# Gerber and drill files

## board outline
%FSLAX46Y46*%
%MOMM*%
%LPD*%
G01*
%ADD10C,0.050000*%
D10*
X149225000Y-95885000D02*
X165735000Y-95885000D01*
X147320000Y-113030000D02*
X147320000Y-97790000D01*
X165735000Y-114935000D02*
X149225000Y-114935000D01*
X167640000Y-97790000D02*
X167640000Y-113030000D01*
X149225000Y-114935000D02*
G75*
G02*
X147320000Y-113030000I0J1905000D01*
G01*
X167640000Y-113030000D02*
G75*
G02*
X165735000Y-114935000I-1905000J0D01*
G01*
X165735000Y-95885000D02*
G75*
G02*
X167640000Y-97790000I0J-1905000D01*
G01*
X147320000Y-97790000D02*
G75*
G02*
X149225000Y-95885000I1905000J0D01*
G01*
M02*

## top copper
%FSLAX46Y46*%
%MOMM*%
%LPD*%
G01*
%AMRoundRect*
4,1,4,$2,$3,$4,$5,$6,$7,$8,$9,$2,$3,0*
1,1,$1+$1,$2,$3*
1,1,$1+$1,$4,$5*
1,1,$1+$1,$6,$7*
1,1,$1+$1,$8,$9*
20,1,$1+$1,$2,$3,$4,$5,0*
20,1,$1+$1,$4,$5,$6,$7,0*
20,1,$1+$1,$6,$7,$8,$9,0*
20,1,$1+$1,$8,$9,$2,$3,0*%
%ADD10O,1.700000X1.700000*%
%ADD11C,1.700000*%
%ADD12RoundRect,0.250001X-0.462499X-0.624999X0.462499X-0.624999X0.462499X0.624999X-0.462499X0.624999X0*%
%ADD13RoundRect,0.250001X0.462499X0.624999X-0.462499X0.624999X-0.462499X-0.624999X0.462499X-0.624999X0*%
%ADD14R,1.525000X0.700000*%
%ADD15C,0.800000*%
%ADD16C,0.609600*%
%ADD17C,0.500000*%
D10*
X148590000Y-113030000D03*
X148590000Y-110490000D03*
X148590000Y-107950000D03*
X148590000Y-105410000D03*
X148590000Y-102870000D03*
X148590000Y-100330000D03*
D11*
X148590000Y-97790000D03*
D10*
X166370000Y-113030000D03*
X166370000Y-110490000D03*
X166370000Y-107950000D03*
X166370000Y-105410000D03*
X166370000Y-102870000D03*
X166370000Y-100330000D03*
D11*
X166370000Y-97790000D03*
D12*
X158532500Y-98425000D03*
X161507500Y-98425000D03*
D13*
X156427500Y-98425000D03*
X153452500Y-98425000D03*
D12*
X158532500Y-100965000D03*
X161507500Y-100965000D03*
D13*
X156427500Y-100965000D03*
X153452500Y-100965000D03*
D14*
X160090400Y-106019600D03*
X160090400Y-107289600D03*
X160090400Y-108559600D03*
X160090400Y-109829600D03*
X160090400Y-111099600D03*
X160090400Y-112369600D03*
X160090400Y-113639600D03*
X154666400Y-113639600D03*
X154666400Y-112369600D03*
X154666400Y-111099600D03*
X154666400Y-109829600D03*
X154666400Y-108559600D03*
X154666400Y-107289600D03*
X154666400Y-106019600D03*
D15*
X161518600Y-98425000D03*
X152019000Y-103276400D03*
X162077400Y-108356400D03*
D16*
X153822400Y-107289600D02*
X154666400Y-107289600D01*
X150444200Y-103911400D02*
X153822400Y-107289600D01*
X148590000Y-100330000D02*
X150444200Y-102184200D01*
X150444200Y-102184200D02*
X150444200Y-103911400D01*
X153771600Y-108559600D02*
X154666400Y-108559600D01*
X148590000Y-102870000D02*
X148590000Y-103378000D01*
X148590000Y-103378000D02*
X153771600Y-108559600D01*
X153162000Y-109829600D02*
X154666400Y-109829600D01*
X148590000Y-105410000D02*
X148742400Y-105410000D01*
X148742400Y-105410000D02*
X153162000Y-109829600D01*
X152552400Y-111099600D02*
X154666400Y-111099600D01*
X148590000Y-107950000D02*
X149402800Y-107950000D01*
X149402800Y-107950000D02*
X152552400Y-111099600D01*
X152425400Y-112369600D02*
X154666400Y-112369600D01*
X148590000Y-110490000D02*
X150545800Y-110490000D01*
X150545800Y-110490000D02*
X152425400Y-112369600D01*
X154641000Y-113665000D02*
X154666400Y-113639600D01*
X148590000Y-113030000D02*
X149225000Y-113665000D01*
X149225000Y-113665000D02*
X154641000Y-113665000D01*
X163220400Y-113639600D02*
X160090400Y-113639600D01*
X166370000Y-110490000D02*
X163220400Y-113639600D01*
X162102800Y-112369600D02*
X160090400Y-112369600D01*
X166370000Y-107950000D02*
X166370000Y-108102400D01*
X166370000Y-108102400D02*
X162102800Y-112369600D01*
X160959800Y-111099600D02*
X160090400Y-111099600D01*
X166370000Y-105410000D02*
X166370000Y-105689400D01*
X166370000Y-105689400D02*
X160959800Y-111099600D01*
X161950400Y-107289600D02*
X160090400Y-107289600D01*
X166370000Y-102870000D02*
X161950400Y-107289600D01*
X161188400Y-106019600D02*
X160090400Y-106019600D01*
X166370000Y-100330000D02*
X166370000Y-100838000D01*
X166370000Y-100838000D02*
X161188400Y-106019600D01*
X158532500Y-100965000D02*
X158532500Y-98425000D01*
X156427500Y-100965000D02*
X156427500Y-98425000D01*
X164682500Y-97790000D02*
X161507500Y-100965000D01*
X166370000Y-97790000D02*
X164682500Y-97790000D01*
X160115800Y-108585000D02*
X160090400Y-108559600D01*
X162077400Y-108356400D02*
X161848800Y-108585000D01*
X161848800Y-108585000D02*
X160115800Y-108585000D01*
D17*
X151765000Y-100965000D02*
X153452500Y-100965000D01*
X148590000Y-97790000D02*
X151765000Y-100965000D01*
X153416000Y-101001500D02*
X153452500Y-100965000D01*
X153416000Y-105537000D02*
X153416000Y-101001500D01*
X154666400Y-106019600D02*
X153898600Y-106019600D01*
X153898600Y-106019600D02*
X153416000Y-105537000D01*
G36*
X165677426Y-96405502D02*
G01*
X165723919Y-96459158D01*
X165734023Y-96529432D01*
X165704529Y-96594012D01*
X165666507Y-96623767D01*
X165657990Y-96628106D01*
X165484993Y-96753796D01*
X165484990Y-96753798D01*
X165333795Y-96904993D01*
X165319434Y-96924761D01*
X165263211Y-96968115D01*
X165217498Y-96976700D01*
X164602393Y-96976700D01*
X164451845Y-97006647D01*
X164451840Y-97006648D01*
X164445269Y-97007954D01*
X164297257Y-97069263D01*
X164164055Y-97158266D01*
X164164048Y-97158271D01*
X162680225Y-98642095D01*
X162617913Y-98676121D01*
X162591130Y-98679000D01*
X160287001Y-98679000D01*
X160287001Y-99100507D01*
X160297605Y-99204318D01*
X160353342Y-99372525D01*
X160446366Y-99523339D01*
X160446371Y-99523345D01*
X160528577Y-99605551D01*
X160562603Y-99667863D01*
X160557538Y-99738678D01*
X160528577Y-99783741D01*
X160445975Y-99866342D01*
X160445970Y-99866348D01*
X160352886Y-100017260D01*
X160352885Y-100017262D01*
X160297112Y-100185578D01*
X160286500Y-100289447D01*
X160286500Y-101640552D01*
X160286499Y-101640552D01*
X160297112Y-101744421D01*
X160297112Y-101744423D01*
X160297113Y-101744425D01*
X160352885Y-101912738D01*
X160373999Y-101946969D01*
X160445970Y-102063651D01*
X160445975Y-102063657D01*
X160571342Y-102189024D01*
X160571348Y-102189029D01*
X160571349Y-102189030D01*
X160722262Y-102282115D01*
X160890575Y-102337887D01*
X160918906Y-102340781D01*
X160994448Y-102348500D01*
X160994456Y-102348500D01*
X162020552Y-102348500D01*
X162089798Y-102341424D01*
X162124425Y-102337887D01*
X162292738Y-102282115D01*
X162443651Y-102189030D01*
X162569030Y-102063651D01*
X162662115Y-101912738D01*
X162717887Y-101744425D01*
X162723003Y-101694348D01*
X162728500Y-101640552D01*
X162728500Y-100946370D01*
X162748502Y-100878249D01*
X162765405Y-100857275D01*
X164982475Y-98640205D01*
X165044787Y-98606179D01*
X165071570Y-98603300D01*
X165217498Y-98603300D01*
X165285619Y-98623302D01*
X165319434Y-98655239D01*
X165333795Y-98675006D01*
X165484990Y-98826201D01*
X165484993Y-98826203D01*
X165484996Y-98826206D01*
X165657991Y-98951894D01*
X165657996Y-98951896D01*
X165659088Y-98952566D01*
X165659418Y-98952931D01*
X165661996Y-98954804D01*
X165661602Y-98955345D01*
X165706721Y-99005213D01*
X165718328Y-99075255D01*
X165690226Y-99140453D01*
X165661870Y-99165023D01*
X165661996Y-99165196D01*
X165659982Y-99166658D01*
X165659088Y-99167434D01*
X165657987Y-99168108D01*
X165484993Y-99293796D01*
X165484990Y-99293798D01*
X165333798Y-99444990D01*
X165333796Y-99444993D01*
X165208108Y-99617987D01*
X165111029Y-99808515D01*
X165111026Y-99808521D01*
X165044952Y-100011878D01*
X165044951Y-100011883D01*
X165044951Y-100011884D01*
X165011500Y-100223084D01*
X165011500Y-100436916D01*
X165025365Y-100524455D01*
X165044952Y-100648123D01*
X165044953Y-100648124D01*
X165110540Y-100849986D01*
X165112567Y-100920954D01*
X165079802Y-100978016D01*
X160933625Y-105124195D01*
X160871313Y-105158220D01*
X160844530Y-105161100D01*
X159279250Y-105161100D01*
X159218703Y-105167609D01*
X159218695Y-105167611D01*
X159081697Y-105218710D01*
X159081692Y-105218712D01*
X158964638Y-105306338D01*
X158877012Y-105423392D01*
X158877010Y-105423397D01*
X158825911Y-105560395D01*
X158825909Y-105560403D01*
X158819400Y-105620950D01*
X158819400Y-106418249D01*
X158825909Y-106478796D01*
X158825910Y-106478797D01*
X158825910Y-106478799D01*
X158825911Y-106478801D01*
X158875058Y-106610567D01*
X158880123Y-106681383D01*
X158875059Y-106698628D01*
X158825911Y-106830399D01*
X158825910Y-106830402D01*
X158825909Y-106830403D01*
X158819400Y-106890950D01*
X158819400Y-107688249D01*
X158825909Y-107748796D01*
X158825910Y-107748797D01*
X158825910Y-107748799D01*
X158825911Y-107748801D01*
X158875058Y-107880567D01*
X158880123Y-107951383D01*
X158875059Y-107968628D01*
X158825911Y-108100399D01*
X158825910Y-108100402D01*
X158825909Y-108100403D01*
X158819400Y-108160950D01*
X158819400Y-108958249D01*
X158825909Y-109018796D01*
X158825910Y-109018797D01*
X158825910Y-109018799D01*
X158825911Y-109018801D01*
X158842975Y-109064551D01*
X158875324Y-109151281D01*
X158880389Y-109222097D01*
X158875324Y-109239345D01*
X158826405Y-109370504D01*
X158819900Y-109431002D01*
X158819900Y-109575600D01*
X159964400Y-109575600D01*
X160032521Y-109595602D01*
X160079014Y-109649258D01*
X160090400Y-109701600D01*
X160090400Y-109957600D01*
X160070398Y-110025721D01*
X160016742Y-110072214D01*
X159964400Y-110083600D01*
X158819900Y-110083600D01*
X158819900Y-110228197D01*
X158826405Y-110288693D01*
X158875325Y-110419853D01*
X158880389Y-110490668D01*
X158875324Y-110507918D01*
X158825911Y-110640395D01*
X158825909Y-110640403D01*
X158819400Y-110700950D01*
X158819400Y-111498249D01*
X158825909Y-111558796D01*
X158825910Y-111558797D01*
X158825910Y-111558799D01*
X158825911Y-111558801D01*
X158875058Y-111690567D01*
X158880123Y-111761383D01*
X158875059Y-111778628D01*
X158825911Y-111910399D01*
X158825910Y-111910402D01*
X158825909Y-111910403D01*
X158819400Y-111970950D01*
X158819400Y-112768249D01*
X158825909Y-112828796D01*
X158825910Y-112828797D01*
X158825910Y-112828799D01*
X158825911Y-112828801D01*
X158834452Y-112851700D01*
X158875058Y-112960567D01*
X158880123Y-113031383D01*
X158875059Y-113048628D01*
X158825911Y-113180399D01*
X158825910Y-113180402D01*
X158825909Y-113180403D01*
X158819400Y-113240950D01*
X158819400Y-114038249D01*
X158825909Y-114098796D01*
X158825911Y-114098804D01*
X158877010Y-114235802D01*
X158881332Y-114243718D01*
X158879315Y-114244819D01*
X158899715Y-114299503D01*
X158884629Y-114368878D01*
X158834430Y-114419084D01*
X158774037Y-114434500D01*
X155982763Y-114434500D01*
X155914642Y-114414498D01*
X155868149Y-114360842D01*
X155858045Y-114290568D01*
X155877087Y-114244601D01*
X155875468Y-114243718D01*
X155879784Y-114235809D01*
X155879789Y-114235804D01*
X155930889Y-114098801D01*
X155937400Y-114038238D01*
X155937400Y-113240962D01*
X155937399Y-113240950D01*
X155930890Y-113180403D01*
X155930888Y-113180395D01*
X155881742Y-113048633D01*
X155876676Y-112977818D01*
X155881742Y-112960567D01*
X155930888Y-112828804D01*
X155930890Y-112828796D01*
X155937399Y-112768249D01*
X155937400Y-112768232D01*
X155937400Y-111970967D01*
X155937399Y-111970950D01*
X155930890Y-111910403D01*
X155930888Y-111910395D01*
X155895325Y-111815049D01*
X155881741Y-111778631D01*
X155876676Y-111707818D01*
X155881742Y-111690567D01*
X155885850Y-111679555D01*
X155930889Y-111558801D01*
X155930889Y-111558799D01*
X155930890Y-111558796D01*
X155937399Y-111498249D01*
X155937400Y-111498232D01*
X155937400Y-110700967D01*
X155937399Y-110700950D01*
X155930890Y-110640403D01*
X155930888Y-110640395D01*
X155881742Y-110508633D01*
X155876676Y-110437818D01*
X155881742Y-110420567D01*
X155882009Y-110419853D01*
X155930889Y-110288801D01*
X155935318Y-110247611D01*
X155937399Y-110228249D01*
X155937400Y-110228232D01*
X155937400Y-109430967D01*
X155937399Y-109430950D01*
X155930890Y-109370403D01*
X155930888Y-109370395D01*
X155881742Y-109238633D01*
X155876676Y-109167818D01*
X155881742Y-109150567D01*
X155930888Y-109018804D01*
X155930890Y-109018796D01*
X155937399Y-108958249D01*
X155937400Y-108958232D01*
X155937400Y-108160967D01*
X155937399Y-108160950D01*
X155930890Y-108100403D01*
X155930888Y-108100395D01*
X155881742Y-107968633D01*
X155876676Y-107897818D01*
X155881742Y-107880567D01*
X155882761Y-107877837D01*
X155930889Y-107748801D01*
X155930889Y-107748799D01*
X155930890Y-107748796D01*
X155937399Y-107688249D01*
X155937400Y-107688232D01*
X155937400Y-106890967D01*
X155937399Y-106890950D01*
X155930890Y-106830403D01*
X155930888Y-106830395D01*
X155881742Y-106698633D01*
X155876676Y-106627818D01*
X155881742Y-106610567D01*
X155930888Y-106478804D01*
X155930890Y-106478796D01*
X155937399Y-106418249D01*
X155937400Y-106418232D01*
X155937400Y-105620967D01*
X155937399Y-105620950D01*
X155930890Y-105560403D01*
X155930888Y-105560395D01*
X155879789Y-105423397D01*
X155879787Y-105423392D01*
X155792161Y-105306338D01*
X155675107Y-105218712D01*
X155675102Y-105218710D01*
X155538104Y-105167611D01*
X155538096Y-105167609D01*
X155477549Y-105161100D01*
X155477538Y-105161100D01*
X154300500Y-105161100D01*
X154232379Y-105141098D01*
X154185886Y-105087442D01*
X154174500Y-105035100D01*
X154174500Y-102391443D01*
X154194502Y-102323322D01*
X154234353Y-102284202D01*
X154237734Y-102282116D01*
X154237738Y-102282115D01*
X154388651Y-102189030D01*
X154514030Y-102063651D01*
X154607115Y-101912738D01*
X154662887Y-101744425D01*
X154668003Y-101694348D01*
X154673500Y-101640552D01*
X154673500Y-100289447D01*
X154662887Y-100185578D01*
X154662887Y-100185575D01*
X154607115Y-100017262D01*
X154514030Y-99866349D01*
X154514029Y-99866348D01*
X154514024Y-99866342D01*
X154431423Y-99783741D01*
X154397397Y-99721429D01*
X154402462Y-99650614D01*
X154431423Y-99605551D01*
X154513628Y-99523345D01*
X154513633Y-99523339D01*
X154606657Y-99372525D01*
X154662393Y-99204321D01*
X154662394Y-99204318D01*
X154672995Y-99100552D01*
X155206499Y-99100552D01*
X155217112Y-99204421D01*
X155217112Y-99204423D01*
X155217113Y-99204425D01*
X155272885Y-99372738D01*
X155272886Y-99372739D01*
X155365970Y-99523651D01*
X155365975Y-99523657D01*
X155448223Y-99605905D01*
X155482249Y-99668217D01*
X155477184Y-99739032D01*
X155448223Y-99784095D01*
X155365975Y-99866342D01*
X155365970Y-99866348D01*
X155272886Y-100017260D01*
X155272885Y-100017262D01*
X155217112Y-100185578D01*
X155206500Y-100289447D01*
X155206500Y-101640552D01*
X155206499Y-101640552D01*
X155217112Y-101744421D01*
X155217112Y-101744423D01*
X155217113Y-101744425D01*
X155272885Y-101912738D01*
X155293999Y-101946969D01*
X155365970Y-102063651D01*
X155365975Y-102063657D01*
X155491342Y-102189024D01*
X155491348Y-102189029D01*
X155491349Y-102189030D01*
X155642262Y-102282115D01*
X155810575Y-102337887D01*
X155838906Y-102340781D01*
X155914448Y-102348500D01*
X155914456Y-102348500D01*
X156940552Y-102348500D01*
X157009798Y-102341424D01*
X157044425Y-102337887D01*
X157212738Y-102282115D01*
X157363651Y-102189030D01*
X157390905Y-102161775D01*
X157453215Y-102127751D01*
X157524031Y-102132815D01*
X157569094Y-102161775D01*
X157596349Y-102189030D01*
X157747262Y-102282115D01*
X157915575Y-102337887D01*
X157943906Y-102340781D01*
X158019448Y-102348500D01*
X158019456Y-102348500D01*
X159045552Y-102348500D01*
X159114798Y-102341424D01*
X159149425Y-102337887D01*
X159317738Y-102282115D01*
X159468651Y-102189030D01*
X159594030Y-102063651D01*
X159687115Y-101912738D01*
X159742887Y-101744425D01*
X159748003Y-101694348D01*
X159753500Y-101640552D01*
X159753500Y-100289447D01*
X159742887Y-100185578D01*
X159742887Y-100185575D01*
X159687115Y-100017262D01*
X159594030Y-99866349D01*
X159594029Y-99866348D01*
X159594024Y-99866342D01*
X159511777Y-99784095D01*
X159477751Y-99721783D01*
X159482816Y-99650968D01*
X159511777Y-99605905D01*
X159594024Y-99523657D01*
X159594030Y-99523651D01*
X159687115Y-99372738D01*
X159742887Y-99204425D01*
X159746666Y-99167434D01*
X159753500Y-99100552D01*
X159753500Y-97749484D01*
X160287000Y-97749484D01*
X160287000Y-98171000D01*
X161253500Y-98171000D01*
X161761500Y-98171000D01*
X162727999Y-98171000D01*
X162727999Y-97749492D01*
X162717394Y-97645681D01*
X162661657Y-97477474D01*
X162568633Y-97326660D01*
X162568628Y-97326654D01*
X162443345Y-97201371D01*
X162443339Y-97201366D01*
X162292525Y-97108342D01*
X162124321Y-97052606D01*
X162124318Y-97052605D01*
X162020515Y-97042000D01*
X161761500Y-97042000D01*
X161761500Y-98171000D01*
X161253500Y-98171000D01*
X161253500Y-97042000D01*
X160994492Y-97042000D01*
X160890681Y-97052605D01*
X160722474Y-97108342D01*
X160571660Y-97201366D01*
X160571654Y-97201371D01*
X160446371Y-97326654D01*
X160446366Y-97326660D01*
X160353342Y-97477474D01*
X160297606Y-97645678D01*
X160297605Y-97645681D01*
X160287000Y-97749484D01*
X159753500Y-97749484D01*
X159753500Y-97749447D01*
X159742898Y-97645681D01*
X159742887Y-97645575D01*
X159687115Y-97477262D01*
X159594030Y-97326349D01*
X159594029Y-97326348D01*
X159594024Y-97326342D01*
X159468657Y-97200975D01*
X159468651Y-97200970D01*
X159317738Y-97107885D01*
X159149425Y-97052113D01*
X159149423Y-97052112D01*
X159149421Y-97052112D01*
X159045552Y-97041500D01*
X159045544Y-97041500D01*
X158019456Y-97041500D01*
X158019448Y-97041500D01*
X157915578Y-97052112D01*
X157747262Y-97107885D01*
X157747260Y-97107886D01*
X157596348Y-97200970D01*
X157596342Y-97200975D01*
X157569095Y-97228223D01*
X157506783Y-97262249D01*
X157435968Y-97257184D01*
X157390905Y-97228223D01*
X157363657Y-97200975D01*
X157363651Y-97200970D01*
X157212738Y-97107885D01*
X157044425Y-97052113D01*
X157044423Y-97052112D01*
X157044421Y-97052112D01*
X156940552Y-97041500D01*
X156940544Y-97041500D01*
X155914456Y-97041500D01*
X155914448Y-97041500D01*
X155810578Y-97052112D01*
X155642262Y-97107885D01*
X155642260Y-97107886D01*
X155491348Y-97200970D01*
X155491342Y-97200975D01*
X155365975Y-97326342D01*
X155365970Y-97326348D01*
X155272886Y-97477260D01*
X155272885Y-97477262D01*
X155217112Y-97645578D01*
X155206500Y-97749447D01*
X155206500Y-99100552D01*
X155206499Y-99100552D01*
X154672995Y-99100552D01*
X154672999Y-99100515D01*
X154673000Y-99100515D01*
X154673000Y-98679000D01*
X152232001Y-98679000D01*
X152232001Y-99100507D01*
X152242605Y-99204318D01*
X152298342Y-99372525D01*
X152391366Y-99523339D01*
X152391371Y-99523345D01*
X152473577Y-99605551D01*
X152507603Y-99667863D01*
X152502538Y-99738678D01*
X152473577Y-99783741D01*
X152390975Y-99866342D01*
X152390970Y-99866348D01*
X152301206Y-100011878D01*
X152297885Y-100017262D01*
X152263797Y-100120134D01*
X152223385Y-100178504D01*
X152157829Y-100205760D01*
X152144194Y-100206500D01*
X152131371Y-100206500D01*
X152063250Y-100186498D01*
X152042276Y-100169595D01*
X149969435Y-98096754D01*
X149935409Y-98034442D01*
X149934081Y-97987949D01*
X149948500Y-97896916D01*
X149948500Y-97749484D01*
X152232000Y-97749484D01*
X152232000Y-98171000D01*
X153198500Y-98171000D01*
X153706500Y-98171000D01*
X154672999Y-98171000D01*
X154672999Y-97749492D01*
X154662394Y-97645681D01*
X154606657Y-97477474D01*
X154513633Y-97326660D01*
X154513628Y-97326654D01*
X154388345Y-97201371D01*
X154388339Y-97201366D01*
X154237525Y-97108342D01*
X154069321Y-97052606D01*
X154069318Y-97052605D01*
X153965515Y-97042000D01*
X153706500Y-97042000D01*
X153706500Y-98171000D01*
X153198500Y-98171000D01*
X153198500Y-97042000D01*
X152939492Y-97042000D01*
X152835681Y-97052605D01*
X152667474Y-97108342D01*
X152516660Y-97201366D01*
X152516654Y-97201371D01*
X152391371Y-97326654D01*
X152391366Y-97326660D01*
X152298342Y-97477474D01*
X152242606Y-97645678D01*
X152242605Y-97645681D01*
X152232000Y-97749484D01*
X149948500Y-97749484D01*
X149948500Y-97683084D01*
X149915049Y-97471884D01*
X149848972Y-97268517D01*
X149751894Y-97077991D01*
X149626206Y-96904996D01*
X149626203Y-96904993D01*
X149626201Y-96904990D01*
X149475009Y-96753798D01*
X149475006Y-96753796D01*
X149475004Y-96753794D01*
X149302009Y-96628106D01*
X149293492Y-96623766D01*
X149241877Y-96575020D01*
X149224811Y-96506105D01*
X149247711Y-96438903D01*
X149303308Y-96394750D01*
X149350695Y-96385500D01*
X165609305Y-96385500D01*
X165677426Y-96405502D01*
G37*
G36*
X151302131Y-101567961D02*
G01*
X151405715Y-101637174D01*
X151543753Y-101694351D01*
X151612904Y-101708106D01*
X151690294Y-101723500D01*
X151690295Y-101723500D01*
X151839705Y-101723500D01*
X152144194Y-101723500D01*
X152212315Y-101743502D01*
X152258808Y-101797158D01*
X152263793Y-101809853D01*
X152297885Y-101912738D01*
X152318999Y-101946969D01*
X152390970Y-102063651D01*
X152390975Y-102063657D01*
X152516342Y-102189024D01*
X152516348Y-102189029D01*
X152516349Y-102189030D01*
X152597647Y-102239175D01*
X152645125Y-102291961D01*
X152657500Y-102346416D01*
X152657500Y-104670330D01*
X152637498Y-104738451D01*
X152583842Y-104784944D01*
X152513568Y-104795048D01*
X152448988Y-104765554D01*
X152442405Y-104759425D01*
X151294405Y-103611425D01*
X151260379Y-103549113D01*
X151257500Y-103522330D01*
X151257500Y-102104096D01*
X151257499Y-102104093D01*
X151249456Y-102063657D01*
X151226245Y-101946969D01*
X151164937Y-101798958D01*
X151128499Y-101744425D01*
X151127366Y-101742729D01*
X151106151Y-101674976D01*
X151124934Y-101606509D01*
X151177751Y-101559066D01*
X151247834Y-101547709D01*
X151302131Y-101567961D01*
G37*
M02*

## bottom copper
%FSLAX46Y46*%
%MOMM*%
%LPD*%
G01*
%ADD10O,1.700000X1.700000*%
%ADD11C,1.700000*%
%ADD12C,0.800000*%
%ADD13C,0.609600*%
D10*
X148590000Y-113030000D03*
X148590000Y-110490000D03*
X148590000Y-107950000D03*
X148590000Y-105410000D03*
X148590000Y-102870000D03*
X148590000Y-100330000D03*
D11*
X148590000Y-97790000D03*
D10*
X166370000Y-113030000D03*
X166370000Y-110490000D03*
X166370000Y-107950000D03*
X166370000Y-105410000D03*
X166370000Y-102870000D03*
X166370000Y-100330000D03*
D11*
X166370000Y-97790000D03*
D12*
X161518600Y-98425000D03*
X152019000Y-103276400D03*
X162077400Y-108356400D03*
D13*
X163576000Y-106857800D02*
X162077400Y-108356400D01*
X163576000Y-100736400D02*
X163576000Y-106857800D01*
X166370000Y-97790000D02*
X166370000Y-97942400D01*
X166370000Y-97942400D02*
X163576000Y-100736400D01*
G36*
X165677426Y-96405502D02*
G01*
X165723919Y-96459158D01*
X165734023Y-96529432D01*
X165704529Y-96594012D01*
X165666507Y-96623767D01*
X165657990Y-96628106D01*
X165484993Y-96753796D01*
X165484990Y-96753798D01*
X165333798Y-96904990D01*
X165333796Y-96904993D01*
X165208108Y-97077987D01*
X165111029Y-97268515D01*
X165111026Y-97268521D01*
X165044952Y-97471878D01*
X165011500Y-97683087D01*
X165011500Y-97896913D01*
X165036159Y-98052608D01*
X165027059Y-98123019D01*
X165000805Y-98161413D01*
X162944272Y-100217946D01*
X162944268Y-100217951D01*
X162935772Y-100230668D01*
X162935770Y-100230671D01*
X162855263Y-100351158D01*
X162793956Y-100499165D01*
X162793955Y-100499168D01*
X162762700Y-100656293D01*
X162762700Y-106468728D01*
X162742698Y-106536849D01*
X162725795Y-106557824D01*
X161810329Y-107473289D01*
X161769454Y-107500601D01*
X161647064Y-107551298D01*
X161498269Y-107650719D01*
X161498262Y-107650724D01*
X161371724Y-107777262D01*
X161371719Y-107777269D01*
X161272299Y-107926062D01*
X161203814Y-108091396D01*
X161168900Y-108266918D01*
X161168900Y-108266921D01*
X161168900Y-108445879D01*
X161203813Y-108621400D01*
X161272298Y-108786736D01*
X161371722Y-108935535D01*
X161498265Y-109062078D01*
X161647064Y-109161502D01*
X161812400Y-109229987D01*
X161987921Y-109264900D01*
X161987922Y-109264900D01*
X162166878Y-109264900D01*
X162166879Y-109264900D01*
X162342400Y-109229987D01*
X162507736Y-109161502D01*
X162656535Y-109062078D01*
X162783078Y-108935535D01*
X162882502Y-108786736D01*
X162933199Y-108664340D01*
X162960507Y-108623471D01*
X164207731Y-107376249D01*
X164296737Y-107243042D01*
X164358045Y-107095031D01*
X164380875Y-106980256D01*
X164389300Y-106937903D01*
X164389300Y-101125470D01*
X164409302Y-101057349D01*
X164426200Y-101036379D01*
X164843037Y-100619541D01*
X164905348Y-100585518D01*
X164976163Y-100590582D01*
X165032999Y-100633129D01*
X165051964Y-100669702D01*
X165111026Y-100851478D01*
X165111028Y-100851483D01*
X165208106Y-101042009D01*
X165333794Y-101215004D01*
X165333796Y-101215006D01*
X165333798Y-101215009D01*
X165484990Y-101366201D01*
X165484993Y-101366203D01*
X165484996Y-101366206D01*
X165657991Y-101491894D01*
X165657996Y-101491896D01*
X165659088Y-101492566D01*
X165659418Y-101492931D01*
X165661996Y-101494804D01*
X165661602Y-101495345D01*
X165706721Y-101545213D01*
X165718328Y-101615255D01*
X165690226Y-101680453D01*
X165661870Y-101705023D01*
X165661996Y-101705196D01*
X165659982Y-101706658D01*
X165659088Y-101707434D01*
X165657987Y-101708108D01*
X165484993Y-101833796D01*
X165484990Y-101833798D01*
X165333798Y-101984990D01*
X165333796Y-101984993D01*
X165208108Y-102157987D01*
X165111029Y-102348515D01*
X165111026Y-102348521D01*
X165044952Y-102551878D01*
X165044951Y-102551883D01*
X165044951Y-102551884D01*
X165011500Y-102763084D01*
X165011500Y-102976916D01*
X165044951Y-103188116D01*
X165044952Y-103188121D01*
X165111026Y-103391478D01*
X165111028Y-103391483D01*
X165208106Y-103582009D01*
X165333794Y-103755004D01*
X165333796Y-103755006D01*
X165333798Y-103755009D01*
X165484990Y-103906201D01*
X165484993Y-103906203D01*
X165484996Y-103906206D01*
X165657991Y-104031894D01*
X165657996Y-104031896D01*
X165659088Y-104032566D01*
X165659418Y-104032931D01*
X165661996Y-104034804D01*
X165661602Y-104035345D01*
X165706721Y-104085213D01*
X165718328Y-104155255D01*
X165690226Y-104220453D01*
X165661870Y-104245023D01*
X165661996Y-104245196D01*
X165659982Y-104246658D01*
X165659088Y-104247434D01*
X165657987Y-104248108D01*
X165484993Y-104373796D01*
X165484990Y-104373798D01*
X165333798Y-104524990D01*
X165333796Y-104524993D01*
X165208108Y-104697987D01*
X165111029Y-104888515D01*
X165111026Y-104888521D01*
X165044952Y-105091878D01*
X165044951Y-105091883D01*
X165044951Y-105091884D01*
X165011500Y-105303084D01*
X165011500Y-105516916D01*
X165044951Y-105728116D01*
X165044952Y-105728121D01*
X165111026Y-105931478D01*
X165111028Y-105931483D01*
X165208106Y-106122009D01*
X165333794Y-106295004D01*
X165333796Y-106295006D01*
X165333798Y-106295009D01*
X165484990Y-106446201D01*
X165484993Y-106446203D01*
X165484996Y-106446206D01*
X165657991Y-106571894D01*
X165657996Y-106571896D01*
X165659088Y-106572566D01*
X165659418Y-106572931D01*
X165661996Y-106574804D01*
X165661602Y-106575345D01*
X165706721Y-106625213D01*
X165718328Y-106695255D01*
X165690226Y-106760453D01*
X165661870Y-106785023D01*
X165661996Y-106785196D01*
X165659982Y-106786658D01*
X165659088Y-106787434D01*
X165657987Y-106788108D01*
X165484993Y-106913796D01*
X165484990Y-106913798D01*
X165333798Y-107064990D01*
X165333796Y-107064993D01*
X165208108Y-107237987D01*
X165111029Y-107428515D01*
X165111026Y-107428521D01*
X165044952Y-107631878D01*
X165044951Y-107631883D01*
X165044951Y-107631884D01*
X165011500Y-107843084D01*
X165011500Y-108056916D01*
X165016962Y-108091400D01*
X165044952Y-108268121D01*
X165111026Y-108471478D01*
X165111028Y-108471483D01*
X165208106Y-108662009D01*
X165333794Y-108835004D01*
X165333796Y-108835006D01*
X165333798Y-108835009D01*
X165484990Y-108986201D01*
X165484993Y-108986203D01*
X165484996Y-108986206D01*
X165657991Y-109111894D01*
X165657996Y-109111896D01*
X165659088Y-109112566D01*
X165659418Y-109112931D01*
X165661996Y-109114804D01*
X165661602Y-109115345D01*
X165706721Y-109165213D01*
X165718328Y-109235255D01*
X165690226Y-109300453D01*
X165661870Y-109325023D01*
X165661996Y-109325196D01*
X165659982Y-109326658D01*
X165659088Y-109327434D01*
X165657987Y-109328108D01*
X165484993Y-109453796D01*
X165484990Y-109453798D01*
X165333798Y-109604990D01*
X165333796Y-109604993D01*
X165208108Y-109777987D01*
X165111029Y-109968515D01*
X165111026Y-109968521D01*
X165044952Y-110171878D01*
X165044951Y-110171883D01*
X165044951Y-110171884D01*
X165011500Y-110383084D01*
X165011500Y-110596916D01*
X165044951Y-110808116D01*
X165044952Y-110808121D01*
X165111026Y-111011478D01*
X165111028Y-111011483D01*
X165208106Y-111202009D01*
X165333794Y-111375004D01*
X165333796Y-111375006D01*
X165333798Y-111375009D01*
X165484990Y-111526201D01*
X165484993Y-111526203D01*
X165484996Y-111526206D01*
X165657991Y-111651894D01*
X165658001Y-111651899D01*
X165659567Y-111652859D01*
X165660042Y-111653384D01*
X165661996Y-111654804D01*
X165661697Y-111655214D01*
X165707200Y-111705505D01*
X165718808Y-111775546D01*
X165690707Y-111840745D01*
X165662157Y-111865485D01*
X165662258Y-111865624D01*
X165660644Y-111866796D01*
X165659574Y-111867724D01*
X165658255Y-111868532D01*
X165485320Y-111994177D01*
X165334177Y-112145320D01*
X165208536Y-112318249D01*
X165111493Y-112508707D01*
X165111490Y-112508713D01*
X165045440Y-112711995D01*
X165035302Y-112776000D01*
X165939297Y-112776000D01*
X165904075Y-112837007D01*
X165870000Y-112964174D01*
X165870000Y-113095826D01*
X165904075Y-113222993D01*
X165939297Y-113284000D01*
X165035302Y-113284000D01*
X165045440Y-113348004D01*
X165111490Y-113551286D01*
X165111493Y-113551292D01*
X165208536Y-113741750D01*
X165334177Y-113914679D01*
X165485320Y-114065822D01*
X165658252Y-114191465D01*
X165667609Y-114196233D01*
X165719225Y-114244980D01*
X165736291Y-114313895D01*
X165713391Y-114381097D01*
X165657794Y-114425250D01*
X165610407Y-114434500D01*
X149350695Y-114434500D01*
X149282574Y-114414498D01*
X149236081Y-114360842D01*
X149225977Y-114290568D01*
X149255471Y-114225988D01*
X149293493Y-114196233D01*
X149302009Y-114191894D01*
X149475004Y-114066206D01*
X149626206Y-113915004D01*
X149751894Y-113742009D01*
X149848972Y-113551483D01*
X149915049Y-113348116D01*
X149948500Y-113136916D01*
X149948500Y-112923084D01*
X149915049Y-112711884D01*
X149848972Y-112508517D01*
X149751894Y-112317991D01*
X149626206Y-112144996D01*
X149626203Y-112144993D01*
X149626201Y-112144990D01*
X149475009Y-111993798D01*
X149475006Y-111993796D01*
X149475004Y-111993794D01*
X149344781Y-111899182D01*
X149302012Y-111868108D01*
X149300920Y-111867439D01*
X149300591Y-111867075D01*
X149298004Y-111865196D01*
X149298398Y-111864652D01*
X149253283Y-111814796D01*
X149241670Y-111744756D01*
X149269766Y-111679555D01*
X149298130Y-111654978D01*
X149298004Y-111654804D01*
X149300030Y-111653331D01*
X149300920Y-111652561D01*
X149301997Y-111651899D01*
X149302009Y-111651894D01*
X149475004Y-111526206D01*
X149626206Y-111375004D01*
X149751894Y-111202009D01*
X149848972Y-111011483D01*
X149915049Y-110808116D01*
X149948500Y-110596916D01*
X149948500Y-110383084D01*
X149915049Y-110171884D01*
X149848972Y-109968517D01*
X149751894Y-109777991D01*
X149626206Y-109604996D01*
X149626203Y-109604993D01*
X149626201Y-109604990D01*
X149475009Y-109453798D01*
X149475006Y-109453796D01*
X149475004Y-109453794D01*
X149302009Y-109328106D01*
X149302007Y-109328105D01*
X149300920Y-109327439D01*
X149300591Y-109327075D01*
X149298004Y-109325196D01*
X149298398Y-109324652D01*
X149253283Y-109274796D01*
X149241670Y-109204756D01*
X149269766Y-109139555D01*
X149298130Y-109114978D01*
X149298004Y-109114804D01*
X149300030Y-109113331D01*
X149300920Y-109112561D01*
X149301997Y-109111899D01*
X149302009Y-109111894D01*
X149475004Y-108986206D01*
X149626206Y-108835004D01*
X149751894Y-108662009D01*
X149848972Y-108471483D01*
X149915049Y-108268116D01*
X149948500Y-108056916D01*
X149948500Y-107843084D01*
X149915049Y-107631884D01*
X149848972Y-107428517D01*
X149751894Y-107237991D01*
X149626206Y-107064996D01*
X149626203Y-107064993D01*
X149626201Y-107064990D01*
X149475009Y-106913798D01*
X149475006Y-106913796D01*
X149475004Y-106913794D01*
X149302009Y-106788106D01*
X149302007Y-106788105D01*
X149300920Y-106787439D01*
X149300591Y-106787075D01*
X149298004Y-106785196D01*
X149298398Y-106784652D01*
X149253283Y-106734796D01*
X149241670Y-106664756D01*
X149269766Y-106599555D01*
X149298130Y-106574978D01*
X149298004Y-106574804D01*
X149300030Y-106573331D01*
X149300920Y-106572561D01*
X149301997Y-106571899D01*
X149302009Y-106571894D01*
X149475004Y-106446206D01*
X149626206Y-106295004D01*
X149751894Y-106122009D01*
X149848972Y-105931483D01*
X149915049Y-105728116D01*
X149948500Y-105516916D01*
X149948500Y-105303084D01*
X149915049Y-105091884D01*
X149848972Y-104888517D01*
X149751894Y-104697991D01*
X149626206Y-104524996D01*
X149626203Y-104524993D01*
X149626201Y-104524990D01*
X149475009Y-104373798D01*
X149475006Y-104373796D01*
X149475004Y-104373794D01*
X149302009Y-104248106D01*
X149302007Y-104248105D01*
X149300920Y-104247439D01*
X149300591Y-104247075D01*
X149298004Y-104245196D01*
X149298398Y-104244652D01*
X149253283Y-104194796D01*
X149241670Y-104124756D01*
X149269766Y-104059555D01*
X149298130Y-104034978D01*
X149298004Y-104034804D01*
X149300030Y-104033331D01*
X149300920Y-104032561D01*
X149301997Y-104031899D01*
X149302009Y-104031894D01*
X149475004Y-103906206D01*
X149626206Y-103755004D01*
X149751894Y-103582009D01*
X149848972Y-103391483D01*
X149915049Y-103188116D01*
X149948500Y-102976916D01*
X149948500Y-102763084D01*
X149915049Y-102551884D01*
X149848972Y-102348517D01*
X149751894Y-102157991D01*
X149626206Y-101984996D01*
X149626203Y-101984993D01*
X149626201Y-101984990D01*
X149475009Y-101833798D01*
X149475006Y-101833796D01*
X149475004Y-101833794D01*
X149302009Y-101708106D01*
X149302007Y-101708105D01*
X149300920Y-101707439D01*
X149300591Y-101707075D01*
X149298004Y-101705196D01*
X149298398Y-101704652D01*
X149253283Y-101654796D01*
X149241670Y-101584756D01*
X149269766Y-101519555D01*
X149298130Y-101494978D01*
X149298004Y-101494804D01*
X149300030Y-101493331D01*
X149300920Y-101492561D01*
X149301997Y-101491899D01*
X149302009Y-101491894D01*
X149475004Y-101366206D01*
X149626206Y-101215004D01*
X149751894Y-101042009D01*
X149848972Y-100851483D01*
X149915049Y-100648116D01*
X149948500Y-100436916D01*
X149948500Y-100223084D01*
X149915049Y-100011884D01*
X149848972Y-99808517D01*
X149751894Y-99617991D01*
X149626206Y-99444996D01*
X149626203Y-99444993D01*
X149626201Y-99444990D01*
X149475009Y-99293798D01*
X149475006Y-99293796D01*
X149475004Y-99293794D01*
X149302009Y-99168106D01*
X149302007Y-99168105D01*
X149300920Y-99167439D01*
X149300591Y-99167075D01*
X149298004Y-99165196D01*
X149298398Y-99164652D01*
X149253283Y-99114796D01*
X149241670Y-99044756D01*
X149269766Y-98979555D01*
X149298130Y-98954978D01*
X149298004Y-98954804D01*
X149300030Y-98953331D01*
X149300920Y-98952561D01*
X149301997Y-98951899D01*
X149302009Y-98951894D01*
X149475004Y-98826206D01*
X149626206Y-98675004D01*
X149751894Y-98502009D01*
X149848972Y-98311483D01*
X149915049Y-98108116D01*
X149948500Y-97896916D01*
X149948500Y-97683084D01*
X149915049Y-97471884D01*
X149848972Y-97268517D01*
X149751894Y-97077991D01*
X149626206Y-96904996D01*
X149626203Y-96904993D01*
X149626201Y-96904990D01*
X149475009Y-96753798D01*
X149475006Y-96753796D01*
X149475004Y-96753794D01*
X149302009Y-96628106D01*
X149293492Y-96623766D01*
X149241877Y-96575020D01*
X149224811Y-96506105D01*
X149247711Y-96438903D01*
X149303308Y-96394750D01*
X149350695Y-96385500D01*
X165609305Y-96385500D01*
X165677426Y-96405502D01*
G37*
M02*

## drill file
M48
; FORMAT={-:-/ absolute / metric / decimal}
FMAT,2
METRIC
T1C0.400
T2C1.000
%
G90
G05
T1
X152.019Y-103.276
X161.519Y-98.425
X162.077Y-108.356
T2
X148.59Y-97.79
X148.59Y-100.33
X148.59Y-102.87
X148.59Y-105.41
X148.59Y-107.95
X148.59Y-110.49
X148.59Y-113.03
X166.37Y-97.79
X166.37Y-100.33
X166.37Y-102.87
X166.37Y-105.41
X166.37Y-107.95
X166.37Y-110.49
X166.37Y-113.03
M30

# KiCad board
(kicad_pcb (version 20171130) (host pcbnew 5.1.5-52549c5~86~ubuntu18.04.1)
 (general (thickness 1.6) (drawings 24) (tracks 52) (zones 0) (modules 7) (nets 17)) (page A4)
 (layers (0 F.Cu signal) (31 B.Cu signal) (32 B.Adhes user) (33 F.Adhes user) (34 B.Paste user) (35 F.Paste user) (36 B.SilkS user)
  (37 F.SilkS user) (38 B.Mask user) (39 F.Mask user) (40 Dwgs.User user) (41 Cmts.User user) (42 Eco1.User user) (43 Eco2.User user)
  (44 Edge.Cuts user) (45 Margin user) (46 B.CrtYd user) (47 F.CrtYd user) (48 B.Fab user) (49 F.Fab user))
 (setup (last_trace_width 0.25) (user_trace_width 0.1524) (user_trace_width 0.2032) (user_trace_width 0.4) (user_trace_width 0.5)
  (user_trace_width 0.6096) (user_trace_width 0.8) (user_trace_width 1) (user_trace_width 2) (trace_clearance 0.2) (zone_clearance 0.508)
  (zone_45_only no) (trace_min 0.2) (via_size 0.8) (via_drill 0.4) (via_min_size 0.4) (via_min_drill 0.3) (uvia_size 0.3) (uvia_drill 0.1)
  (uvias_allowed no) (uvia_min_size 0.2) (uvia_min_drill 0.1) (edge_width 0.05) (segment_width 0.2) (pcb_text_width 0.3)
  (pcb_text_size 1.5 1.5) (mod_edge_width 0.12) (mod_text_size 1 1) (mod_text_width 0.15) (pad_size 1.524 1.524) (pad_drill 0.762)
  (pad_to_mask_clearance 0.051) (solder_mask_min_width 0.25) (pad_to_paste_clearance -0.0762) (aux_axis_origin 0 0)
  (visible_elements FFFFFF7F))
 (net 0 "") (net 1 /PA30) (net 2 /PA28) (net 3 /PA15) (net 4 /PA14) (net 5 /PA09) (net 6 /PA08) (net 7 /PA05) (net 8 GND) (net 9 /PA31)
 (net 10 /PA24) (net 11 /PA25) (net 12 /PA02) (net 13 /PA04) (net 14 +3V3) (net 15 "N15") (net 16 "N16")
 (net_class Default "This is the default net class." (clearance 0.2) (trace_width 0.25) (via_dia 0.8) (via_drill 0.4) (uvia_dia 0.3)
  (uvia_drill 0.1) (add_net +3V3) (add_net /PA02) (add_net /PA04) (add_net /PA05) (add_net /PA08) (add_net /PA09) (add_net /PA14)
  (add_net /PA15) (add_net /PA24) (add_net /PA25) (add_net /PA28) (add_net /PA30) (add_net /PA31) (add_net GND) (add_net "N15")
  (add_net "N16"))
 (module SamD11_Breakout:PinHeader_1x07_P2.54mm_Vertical (layer F.Cu) (at 148.59 97.79)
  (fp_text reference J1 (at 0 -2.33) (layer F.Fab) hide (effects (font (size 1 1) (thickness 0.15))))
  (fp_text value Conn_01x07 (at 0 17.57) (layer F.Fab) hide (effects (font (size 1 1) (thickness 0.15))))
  (pad 7 thru_hole oval (at 0 15.24) (size 1.7 1.7) (drill 1) (layers *.Cu *.Mask) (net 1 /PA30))
  (pad 6 thru_hole oval (at 0 12.7) (size 1.7 1.7) (drill 1) (layers *.Cu *.Mask) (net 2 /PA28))
  (pad 5 thru_hole oval (at 0 10.16) (size 1.7 1.7) (drill 1) (layers *.Cu *.Mask) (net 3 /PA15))
  (pad 4 thru_hole oval (at 0 7.62) (size 1.7 1.7) (drill 1) (layers *.Cu *.Mask) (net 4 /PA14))
  (pad 3 thru_hole oval (at 0 5.08) (size 1.7 1.7) (drill 1) (layers *.Cu *.Mask) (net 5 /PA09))
  (pad 2 thru_hole oval (at 0 2.54) (size 1.7 1.7) (drill 1) (layers *.Cu *.Mask) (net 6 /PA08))
  (pad 1 thru_hole circle (at 0 0) (size 1.7 1.7) (drill 1) (layers *.Cu *.Mask) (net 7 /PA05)))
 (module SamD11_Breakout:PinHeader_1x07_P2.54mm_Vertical (layer F.Cu) (at 166.37 97.79)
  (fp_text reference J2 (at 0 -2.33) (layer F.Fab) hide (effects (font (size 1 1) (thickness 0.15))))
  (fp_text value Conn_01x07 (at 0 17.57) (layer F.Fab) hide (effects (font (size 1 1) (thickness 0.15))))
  (pad 7 thru_hole oval (at 0 15.24) (size 1.7 1.7) (drill 1) (layers *.Cu *.Mask) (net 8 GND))
  (pad 6 thru_hole oval (at 0 12.7) (size 1.7 1.7) (drill 1) (layers *.Cu *.Mask) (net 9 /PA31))
  (pad 5 thru_hole oval (at 0 10.16) (size 1.7 1.7) (drill 1) (layers *.Cu *.Mask) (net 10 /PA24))
  (pad 4 thru_hole oval (at 0 7.62) (size 1.7 1.7) (drill 1) (layers *.Cu *.Mask) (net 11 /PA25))
  (pad 3 thru_hole oval (at 0 5.08) (size 1.7 1.7) (drill 1) (layers *.Cu *.Mask) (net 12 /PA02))
  (pad 2 thru_hole oval (at 0 2.54) (size 1.7 1.7) (drill 1) (layers *.Cu *.Mask) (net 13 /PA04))
  (pad 1 thru_hole circle (at 0 0) (size 1.7 1.7) (drill 1) (layers *.Cu *.Mask) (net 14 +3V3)))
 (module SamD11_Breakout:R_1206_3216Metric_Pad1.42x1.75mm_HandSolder (layer F.Cu) (at 160.02 98.425)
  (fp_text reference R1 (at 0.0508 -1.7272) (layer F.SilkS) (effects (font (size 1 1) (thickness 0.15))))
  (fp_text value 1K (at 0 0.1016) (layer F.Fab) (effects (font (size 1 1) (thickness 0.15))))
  (pad 1 smd roundrect (at -1.4875 0) (size 1.425 1.75) (layers F.Cu F.Paste F.Mask) (roundrect_rratio 0.175439) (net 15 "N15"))
  (pad 2 smd roundrect (at 1.4875 0) (size 1.425 1.75) (layers F.Cu F.Paste F.Mask) (roundrect_rratio 0.175439) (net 8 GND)))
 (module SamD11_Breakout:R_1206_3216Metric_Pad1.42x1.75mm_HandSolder (layer F.Cu) (at 154.94 98.425 180)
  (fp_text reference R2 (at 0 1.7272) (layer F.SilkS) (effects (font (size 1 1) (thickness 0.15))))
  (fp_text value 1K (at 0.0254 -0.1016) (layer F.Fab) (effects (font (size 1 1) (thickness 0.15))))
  (pad 1 smd roundrect (at -1.4875 0 180) (size 1.425 1.75) (layers F.Cu F.Paste F.Mask) (roundrect_rratio 0.175439) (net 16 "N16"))
  (pad 2 smd roundrect (at 1.4875 0 180) (size 1.425 1.75) (layers F.Cu F.Paste F.Mask) (roundrect_rratio 0.175439) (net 8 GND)))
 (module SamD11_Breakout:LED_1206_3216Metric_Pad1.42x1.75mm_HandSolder (layer F.Cu) (at 160.02 100.965)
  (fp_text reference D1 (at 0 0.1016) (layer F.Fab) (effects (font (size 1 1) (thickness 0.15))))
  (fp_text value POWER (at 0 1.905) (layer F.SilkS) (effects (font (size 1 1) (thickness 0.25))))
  (pad 1 smd roundrect (at -1.4875 0) (size 1.425 1.75) (layers F.Cu F.Paste F.Mask) (roundrect_rratio 0.175439) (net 15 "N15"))
  (pad 2 smd roundrect (at 1.4875 0) (size 1.425 1.75) (layers F.Cu F.Paste F.Mask) (roundrect_rratio 0.175439) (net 14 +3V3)))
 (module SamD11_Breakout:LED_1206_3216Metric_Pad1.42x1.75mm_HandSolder (layer F.Cu) (at 154.94 100.965 180)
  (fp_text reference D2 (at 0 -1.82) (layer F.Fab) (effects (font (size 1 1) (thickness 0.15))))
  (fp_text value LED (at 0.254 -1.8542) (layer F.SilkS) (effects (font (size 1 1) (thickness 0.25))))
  (pad 1 smd roundrect (at -1.4875 0 180) (size 1.425 1.75) (layers F.Cu F.Paste F.Mask) (roundrect_rratio 0.175439) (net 16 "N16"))
  (pad 2 smd roundrect (at 1.4875 0 180) (size 1.425 1.75) (layers F.Cu F.Paste F.Mask) (roundrect_rratio 0.175439) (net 7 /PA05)))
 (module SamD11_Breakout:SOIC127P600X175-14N (layer F.Cu) (at 157.3784 109.8296)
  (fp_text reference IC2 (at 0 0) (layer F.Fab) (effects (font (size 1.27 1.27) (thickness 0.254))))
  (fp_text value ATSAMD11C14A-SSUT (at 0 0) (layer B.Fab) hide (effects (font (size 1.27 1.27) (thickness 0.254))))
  (pad 14 smd rect (at 2.712 -3.81 90) (size 0.7 1.525) (layers F.Cu F.Paste F.Mask) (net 13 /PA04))
  (pad 13 smd rect (at 2.712 -2.54 90) (size 0.7 1.525) (layers F.Cu F.Paste F.Mask) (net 12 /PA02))
  (pad 12 smd rect (at 2.712 -1.27 90) (size 0.7 1.525) (layers F.Cu F.Paste F.Mask) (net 14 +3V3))
  (pad 11 smd rect (at 2.712 0 90) (size 0.7 1.525) (layers F.Cu F.Paste F.Mask) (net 8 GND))
  (pad 10 smd rect (at 2.712 1.27 90) (size 0.7 1.525) (layers F.Cu F.Paste F.Mask) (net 11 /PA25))
  (pad 9 smd rect (at 2.712 2.54 90) (size 0.7 1.525) (layers F.Cu F.Paste F.Mask) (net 10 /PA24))
  (pad 8 smd rect (at 2.712 3.81 90) (size 0.7 1.525) (layers F.Cu F.Paste F.Mask) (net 9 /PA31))
  (pad 7 smd rect (at -2.712 3.81 90) (size 0.7 1.525) (layers F.Cu F.Paste F.Mask) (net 1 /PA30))
  (pad 6 smd rect (at -2.712 2.54 90) (size 0.7 1.525) (layers F.Cu F.Paste F.Mask) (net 2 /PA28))
  (pad 5 smd rect (at -2.712 1.27 90) (size 0.7 1.525) (layers F.Cu F.Paste F.Mask) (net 3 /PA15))
  (pad 4 smd rect (at -2.712 0 90) (size 0.7 1.525) (layers F.Cu F.Paste F.Mask) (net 4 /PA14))
  (pad 3 smd rect (at -2.712 -1.27 90) (size 0.7 1.525) (layers F.Cu F.Paste F.Mask) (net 5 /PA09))
  (pad 2 smd rect (at -2.712 -2.54 90) (size 0.7 1.525) (layers F.Cu F.Paste F.Mask) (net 6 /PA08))
  (pad 1 smd rect (at -2.712 -3.81 90) (size 0.7 1.525) (layers F.Cu F.Paste F.Mask) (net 7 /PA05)))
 (gr_line (start 149.225 95.885) (end 165.735 95.885) (layer Edge.Cuts) (width 0.05))
 (gr_line (start 147.32 113.03) (end 147.32 97.79) (layer Edge.Cuts) (width 0.05))
 (gr_line (start 165.735 114.935) (end 149.225 114.935) (layer Edge.Cuts) (width 0.05))
 (gr_line (start 167.64 97.79) (end 167.64 113.03) (layer Edge.Cuts) (width 0.05))
 (gr_arc (start 149.225 113.03) (end 147.32 113.03) (angle -90) (layer Edge.Cuts) (width 0.05))
 (gr_arc (start 165.735 113.03) (end 165.735 114.935) (angle -90) (layer Edge.Cuts) (width 0.05))
 (gr_arc (start 165.735 97.79) (end 167.64 97.79) (angle -90) (layer Edge.Cuts) (width 0.05))
 (gr_arc (start 149.225 97.79) (end 149.225 95.885) (angle -90) (layer Edge.Cuts) (width 0.05))
 (via (at 161.5186 98.425) (size 0.8) (drill 0.4) (layers F.Cu B.Cu) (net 8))
 (via (at 152.019 103.2764) (size 0.8) (drill 0.4) (layers F.Cu B.Cu) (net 8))
 (segment (start 153.8224 107.2896) (end 154.6664 107.2896) (width 0.6096) (layer F.Cu) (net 6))
 (segment (start 150.4442 103.9114) (end 153.8224 107.2896) (width 0.6096) (layer F.Cu) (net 6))
 (segment (start 148.59 100.33) (end 150.4442 102.1842) (width 0.6096) (layer F.Cu) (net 6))
 (segment (start 150.4442 102.1842) (end 150.4442 103.9114) (width 0.6096) (layer F.Cu) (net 6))
 (segment (start 153.7716 108.5596) (end 154.6664 108.5596) (width 0.6096) (layer F.Cu) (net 5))
 (segment (start 148.59 102.87) (end 148.59 103.378) (width 0.6096) (layer F.Cu) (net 5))
 (segment (start 148.59 103.378) (end 153.7716 108.5596) (width 0.6096) (layer F.Cu) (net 5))
 (segment (start 153.162 109.8296) (end 154.6664 109.8296) (width 0.6096) (layer F.Cu) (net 4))
 (segment (start 148.59 105.41) (end 148.7424 105.41) (width 0.6096) (layer F.Cu) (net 4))
 (segment (start 148.7424 105.41) (end 153.162 109.8296) (width 0.6096) (layer F.Cu) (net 4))
 (segment (start 152.5524 111.0996) (end 154.6664 111.0996) (width 0.6096) (layer F.Cu) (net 3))
 (segment (start 148.59 107.95) (end 149.4028 107.95) (width 0.6096) (layer F.Cu) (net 3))
 (segment (start 149.4028 107.95) (end 152.5524 111.0996) (width 0.6096) (layer F.Cu) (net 3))
 (segment (start 152.4254 112.3696) (end 154.6664 112.3696) (width 0.6096) (layer F.Cu) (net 2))
 (segment (start 148.59 110.49) (end 150.5458 110.49) (width 0.6096) (layer F.Cu) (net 2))
 (segment (start 150.5458 110.49) (end 152.4254 112.3696) (width 0.6096) (layer F.Cu) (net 2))
 (segment (start 154.641 113.665) (end 154.6664 113.6396) (width 0.6096) (layer F.Cu) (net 1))
 (segment (start 148.59 113.03) (end 149.225 113.665) (width 0.6096) (layer F.Cu) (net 1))
 (segment (start 149.225 113.665) (end 154.641 113.665) (width 0.6096) (layer F.Cu) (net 1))
 (segment (start 163.2204 113.6396) (end 160.0904 113.6396) (width 0.6096) (layer F.Cu) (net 9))
 (segment (start 166.37 110.49) (end 163.2204 113.6396) (width 0.6096) (layer F.Cu) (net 9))
 (segment (start 162.1028 112.3696) (end 160.0904 112.3696) (width 0.6096) (layer F.Cu) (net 10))
 (segment (start 166.37 107.95) (end 166.37 108.1024) (width 0.6096) (layer F.Cu) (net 10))
 (segment (start 166.37 108.1024) (end 162.1028 112.3696) (width 0.6096) (layer F.Cu) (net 10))
 (segment (start 160.9598 111.0996) (end 160.0904 111.0996) (width 0.6096) (layer F.Cu) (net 11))
 (segment (start 166.37 105.41) (end 166.37 105.6894) (width 0.6096) (layer F.Cu) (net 11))
 (segment (start 166.37 105.6894) (end 160.9598 111.0996) (width 0.6096) (layer F.Cu) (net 11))
 (segment (start 161.9504 107.2896) (end 160.0904 107.2896) (width 0.6096) (layer F.Cu) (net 12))
 (segment (start 166.37 102.87) (end 161.9504 107.2896) (width 0.6096) (layer F.Cu) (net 12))
 (segment (start 161.1884 106.0196) (end 160.0904 106.0196) (width 0.6096) (layer F.Cu) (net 13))
 (segment (start 166.37 100.33) (end 166.37 100.838) (width 0.6096) (layer F.Cu) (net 13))
 (segment (start 166.37 100.838) (end 161.1884 106.0196) (width 0.6096) (layer F.Cu) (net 13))
 (segment (start 158.5325 100.965) (end 158.5325 98.425) (width 0.6096) (layer F.Cu) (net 15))
 (segment (start 156.4275 100.965) (end 156.4275 98.425) (width 0.6096) (layer F.Cu) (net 16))
 (segment (start 164.6825 97.79) (end 161.5075 100.965) (width 0.6096) (layer F.Cu) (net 14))
 (segment (start 166.37 97.79) (end 164.6825 97.79) (width 0.6096) (layer F.Cu) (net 14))
 (via (at 162.0774 108.3564) (size 0.8) (drill 0.4) (layers F.Cu B.Cu) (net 14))
 (segment (start 160.1158 108.585) (end 160.0904 108.5596) (width 0.6096) (layer F.Cu) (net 14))
 (segment (start 162.0774 108.3564) (end 161.8488 108.585) (width 0.6096) (layer F.Cu) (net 14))
 (segment (start 161.8488 108.585) (end 160.1158 108.585) (width 0.6096) (layer F.Cu) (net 14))
 (segment (start 163.576 106.8578) (end 162.0774 108.3564) (width 0.6096) (layer B.Cu) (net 14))
 (segment (start 163.576 100.7364) (end 163.576 106.8578) (width 0.6096) (layer B.Cu) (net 14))
 (segment (start 166.37 97.79) (end 166.37 97.9424) (width 0.6096) (layer B.Cu) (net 14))
 (segment (start 166.37 97.9424) (end 163.576 100.7364) (width 0.6096) (layer B.Cu) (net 14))
 (segment (start 151.765 100.965) (end 153.4525 100.965) (width 0.5) (layer F.Cu) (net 7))
 (segment (start 148.59 97.79) (end 151.765 100.965) (width 0.5) (layer F.Cu) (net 7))
 (segment (start 153.416 101.0015) (end 153.4525 100.965) (width 0.5) (layer F.Cu) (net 7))
 (segment (start 153.416 105.537) (end 153.416 101.0015) (width 0.5) (layer F.Cu) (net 7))
 (segment (start 154.6664 106.0196) (end 153.8986 106.0196) (width 0.5) (layer F.Cu) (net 7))
 (segment (start 153.8986 106.0196) (end 153.416 105.537) (width 0.5) (layer F.Cu) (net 7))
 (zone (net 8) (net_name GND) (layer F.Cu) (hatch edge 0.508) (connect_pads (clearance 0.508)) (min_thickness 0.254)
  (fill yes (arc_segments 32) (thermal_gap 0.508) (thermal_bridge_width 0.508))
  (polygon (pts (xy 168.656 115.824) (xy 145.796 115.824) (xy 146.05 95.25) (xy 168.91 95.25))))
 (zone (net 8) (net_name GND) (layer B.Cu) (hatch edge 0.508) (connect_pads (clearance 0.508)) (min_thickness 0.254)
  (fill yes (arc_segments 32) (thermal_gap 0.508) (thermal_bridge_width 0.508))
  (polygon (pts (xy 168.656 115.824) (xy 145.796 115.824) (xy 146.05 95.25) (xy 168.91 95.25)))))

